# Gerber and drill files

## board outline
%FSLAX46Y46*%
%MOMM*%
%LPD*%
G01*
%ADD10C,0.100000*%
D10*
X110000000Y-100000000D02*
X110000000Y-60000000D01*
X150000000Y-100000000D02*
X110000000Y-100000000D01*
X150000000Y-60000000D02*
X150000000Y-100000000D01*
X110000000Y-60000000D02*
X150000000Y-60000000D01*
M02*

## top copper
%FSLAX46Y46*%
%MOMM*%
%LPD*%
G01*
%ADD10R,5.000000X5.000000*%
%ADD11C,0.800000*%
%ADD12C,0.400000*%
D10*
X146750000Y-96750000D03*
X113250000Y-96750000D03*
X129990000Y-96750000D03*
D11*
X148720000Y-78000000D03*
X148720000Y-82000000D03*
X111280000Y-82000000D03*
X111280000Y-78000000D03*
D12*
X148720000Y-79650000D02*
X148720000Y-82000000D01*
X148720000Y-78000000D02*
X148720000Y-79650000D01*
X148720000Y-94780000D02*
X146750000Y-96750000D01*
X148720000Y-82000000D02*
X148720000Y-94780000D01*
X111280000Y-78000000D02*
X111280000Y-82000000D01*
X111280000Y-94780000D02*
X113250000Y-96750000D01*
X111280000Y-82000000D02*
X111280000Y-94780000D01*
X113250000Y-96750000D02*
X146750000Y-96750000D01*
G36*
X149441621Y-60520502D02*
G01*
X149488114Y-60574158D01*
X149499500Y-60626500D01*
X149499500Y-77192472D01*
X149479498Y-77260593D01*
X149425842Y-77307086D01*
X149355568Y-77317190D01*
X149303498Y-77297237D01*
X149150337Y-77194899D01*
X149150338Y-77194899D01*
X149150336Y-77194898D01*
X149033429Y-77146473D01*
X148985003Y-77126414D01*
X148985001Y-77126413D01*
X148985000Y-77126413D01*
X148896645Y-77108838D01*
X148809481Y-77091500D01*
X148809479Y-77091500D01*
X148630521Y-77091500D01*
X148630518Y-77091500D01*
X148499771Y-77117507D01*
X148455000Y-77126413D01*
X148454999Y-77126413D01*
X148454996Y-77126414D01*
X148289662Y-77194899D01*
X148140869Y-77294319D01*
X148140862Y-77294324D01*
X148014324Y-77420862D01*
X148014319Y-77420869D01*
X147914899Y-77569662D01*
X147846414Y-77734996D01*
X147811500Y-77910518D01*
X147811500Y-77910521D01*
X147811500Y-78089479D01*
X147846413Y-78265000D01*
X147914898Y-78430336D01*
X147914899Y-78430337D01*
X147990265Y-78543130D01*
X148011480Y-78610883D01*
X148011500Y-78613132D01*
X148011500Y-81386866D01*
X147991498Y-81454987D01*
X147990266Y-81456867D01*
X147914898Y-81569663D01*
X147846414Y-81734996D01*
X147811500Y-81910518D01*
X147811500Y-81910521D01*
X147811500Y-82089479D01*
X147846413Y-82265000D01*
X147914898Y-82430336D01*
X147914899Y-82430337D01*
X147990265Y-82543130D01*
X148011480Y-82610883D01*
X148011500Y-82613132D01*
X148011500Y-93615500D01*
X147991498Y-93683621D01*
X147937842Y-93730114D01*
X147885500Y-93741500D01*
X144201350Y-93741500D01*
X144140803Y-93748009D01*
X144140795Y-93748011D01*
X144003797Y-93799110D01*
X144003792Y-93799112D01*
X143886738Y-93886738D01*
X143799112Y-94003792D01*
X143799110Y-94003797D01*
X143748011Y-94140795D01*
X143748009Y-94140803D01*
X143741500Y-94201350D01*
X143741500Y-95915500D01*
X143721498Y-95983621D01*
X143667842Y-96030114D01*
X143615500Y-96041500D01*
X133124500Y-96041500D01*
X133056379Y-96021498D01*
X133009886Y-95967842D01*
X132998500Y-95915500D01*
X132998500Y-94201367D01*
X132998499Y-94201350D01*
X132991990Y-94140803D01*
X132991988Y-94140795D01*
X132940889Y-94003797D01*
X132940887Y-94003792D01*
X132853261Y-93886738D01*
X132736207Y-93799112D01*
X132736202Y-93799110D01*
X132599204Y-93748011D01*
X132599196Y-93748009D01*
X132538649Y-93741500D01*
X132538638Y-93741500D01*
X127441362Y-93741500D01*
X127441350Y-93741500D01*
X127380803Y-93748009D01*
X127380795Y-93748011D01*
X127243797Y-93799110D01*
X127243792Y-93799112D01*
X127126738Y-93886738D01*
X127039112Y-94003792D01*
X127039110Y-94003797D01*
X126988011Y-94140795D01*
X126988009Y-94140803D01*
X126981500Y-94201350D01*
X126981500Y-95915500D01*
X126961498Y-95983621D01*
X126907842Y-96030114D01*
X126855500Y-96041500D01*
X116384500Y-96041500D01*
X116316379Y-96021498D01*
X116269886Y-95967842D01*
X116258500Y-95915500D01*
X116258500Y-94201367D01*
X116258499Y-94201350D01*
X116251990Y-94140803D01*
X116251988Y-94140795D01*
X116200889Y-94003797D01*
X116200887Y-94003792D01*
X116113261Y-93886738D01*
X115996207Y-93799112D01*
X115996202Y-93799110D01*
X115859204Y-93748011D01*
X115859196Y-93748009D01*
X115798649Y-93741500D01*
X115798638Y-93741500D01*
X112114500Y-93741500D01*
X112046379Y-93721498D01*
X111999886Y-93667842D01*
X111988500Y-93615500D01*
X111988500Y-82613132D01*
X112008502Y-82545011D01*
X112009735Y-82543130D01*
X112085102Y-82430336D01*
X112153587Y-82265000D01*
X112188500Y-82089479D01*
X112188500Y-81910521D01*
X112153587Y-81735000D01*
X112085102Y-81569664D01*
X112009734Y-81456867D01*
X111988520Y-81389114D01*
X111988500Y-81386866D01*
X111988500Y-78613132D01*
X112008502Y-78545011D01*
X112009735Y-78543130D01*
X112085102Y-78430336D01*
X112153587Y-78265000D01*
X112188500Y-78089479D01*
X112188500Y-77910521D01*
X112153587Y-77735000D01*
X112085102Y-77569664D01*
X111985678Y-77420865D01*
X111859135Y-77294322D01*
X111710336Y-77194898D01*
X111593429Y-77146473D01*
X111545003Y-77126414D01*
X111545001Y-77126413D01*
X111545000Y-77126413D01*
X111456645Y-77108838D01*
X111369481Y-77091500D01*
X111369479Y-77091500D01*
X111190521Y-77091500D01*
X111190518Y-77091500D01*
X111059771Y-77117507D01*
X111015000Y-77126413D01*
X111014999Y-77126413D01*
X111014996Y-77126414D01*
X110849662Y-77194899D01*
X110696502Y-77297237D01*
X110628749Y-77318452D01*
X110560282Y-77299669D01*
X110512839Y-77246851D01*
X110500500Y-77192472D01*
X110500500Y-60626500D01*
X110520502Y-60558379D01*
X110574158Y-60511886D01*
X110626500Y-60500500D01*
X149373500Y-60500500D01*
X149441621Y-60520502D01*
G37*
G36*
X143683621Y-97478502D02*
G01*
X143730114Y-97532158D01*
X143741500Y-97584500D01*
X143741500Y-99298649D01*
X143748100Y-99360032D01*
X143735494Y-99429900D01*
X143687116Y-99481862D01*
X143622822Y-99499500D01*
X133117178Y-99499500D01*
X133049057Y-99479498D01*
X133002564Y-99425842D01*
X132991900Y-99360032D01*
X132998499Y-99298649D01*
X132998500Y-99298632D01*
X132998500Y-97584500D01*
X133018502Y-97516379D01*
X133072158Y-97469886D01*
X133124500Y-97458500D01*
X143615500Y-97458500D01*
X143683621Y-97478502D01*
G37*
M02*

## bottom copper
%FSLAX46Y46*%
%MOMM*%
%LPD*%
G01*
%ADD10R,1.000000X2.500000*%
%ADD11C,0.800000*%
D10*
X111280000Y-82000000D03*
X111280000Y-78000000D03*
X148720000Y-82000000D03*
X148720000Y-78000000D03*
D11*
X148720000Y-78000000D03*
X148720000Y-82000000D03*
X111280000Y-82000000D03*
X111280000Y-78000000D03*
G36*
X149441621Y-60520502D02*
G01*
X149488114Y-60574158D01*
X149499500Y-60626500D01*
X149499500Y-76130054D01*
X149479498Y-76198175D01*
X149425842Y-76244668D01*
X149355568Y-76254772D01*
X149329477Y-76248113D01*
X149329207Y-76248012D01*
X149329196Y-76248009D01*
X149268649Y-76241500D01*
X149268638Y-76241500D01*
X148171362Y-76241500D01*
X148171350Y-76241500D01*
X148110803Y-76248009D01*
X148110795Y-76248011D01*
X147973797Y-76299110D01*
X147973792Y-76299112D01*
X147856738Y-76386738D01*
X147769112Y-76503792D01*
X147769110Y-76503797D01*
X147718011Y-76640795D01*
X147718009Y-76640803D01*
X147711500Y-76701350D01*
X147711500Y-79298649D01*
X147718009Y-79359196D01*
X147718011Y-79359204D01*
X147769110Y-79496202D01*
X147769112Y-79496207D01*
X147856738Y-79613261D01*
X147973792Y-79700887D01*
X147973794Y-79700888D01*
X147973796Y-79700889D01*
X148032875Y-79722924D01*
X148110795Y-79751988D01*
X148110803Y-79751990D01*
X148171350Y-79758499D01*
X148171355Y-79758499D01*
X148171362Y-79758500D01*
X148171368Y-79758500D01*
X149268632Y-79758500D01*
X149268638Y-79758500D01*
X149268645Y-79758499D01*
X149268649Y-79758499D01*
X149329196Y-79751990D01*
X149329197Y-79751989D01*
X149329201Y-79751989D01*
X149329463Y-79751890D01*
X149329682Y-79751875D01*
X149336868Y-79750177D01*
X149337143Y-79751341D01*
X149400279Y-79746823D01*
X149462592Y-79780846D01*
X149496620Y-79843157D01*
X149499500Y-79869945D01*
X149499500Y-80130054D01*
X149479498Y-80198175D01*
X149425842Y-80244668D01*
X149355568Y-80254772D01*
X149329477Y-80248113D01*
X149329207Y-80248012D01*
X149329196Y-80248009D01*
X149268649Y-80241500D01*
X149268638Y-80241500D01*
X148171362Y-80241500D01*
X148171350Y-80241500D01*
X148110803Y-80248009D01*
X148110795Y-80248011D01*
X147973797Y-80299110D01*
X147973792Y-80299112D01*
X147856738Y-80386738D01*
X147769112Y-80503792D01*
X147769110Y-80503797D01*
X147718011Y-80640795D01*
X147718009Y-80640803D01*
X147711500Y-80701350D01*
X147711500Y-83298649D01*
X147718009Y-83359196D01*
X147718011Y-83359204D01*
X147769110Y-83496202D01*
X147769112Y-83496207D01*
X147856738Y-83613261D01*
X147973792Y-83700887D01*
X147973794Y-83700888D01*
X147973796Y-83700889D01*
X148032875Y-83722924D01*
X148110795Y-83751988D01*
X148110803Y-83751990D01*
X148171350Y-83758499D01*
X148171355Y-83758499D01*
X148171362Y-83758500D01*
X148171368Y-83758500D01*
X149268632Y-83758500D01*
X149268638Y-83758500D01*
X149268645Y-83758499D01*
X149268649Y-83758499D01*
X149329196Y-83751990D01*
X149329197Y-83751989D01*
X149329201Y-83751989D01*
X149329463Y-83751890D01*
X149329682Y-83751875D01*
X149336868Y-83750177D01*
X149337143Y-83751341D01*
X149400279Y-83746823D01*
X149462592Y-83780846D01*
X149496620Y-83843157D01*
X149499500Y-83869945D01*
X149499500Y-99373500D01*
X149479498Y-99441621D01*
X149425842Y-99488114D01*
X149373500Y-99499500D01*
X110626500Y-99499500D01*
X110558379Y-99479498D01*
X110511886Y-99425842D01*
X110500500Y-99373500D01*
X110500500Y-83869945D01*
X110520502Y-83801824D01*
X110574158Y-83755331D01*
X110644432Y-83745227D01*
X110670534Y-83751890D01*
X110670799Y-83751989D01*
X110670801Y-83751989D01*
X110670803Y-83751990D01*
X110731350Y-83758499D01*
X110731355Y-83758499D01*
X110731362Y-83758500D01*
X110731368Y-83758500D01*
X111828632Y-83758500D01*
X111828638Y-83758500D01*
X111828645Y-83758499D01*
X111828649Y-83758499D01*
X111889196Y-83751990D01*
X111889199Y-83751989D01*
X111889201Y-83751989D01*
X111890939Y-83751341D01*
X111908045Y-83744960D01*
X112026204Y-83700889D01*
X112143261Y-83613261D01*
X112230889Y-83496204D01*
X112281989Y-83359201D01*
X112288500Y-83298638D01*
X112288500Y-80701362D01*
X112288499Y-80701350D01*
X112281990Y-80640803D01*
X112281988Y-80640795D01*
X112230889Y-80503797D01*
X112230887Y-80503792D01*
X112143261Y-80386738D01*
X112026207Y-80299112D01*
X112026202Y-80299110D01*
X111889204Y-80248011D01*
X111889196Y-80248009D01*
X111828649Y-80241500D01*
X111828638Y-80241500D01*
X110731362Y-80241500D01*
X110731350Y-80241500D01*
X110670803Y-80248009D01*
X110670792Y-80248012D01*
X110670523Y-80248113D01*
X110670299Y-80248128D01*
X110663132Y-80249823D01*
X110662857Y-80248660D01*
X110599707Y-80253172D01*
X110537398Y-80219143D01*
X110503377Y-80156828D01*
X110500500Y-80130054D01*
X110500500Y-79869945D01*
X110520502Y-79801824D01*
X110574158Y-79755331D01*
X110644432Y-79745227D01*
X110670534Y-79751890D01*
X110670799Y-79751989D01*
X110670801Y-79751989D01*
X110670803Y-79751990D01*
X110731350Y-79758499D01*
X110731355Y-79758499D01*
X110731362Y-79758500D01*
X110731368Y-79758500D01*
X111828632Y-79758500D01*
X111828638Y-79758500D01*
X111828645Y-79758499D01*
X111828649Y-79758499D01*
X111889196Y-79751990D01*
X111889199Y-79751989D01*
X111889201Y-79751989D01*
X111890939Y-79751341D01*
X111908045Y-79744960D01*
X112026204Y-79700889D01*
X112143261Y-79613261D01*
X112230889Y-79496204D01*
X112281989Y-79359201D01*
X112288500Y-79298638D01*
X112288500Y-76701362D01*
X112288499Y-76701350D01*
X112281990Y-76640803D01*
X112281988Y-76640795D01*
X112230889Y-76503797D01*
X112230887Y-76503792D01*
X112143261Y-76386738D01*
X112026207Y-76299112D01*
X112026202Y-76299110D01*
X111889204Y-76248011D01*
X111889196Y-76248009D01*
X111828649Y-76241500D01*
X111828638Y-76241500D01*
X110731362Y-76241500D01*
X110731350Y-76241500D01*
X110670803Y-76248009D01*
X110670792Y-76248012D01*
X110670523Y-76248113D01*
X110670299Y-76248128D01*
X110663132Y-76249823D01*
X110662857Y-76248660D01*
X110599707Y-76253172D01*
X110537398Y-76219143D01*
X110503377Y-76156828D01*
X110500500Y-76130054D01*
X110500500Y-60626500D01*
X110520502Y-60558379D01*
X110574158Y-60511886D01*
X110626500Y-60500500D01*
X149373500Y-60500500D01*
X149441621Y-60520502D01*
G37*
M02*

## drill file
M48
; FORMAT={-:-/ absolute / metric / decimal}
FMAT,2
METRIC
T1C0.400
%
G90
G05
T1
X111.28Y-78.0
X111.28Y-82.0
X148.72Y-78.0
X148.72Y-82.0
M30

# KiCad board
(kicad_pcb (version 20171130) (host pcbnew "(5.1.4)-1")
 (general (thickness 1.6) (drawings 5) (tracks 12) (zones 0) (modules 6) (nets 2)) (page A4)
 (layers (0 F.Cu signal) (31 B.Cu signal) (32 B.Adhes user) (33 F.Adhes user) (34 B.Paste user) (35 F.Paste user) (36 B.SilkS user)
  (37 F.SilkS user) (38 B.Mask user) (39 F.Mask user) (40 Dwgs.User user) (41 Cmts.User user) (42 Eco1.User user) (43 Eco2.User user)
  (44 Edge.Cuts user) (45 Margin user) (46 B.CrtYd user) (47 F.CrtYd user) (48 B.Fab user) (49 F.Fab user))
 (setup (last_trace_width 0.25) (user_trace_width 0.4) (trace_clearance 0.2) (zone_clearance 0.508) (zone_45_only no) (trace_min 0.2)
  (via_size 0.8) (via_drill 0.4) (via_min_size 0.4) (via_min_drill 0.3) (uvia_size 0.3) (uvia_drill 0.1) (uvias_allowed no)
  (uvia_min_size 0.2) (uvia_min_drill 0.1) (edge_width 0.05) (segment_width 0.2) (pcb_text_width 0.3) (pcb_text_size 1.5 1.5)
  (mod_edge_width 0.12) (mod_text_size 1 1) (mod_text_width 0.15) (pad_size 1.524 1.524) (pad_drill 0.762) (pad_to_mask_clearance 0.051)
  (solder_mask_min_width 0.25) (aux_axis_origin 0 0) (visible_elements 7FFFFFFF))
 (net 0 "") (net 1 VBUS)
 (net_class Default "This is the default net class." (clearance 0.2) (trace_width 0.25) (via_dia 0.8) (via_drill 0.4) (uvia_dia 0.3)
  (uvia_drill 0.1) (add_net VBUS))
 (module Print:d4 (layer F.Cu) (at 130 80 90)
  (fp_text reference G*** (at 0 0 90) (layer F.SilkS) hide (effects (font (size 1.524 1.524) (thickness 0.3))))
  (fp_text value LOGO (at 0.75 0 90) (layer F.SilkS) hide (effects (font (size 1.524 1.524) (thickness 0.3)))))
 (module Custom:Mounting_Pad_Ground (layer F.Cu) (at 146.75 96.75)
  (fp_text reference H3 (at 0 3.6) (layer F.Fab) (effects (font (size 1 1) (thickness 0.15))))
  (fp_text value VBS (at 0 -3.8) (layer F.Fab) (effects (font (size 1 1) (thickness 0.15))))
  (pad 1 smd rect (at 0 0) (size 5 5) (layers F.Cu F.Paste F.Mask) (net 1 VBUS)))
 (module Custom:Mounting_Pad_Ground (layer F.Cu) (at 113.25 96.75)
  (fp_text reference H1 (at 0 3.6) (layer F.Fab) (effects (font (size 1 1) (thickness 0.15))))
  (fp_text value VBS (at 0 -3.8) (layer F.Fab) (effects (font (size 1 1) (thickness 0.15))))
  (pad 1 smd rect (at 0 0) (size 5 5) (layers F.Cu F.Paste F.Mask) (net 1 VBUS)))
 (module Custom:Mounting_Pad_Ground (layer F.Cu) (at 129.99 96.75)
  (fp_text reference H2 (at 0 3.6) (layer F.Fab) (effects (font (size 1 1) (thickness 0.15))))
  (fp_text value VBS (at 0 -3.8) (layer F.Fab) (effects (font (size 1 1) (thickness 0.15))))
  (pad 1 smd rect (at 0 0) (size 5 5) (layers F.Cu F.Paste F.Mask) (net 1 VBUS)))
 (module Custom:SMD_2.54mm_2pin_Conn (layer B.Cu) (at 113.1 80 90)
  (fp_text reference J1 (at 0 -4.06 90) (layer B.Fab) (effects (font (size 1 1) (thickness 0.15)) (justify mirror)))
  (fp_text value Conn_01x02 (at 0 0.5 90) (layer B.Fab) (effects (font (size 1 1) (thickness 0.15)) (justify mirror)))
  (pad 1 smd rect (at -2 -1.82 90) (size 2.5 1) (layers B.Cu B.Paste B.Mask) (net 1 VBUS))
  (pad 2 smd rect (at 2 -1.82 90) (size 2.5 1) (layers B.Cu B.Paste B.Mask) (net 1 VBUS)))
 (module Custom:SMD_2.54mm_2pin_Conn (layer B.Cu) (at 150.54 80 90)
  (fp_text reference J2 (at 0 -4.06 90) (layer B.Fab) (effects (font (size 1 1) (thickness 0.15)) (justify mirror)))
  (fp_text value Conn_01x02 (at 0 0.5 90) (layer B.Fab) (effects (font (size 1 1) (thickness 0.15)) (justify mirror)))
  (pad 1 smd rect (at -2 -1.82 90) (size 2.5 1) (layers B.Cu B.Paste B.Mask) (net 1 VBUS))
  (pad 2 smd rect (at 2 -1.82 90) (size 2.5 1) (layers B.Cu B.Paste B.Mask) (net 1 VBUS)))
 (gr_line (start 110 100) (end 110 60) (layer Edge.Cuts) (width 0.1))
 (gr_line (start 150 100) (end 110 100) (layer Edge.Cuts) (width 0.1))
 (gr_line (start 150 60) (end 150 100) (layer Edge.Cuts) (width 0.1))
 (gr_line (start 110 60) (end 150 60) (layer Edge.Cuts) (width 0.1))
 (via (at 148.72 78) (size 0.8) (drill 0.4) (layers F.Cu B.Cu) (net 1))
 (via (at 148.72 82) (size 0.8) (drill 0.4) (layers F.Cu B.Cu) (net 1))
 (via (at 111.28 82) (size 0.8) (drill 0.4) (layers F.Cu B.Cu) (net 1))
 (via (at 111.28 78) (size 0.8) (drill 0.4) (layers F.Cu B.Cu) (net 1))
 (segment (start 148.72 79.65) (end 148.72 82) (width 0.4) (layer F.Cu) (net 1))
 (segment (start 148.72 78) (end 148.72 79.65) (width 0.4) (layer F.Cu) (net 1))
 (segment (start 148.72 94.78) (end 146.75 96.75) (width 0.4) (layer F.Cu) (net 1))
 (segment (start 148.72 82) (end 148.72 94.78) (width 0.4) (layer F.Cu) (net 1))
 (segment (start 111.28 78) (end 111.28 82) (width 0.4) (layer F.Cu) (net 1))
 (segment (start 111.28 94.78) (end 113.25 96.75) (width 0.4) (layer F.Cu) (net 1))
 (segment (start 111.28 82) (end 111.28 94.78) (width 0.4) (layer F.Cu) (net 1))
 (segment (start 113.25 96.75) (end 146.75 96.75) (width 0.4) (layer F.Cu) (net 1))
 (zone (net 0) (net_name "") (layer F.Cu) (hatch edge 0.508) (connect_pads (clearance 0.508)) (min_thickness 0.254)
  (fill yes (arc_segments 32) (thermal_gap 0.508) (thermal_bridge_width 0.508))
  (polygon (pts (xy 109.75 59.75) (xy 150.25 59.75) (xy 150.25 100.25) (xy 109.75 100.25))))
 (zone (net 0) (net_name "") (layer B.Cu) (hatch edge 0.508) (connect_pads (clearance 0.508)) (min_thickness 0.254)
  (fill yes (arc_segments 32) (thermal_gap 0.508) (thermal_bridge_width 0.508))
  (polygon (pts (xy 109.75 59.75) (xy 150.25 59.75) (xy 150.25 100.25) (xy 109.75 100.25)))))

